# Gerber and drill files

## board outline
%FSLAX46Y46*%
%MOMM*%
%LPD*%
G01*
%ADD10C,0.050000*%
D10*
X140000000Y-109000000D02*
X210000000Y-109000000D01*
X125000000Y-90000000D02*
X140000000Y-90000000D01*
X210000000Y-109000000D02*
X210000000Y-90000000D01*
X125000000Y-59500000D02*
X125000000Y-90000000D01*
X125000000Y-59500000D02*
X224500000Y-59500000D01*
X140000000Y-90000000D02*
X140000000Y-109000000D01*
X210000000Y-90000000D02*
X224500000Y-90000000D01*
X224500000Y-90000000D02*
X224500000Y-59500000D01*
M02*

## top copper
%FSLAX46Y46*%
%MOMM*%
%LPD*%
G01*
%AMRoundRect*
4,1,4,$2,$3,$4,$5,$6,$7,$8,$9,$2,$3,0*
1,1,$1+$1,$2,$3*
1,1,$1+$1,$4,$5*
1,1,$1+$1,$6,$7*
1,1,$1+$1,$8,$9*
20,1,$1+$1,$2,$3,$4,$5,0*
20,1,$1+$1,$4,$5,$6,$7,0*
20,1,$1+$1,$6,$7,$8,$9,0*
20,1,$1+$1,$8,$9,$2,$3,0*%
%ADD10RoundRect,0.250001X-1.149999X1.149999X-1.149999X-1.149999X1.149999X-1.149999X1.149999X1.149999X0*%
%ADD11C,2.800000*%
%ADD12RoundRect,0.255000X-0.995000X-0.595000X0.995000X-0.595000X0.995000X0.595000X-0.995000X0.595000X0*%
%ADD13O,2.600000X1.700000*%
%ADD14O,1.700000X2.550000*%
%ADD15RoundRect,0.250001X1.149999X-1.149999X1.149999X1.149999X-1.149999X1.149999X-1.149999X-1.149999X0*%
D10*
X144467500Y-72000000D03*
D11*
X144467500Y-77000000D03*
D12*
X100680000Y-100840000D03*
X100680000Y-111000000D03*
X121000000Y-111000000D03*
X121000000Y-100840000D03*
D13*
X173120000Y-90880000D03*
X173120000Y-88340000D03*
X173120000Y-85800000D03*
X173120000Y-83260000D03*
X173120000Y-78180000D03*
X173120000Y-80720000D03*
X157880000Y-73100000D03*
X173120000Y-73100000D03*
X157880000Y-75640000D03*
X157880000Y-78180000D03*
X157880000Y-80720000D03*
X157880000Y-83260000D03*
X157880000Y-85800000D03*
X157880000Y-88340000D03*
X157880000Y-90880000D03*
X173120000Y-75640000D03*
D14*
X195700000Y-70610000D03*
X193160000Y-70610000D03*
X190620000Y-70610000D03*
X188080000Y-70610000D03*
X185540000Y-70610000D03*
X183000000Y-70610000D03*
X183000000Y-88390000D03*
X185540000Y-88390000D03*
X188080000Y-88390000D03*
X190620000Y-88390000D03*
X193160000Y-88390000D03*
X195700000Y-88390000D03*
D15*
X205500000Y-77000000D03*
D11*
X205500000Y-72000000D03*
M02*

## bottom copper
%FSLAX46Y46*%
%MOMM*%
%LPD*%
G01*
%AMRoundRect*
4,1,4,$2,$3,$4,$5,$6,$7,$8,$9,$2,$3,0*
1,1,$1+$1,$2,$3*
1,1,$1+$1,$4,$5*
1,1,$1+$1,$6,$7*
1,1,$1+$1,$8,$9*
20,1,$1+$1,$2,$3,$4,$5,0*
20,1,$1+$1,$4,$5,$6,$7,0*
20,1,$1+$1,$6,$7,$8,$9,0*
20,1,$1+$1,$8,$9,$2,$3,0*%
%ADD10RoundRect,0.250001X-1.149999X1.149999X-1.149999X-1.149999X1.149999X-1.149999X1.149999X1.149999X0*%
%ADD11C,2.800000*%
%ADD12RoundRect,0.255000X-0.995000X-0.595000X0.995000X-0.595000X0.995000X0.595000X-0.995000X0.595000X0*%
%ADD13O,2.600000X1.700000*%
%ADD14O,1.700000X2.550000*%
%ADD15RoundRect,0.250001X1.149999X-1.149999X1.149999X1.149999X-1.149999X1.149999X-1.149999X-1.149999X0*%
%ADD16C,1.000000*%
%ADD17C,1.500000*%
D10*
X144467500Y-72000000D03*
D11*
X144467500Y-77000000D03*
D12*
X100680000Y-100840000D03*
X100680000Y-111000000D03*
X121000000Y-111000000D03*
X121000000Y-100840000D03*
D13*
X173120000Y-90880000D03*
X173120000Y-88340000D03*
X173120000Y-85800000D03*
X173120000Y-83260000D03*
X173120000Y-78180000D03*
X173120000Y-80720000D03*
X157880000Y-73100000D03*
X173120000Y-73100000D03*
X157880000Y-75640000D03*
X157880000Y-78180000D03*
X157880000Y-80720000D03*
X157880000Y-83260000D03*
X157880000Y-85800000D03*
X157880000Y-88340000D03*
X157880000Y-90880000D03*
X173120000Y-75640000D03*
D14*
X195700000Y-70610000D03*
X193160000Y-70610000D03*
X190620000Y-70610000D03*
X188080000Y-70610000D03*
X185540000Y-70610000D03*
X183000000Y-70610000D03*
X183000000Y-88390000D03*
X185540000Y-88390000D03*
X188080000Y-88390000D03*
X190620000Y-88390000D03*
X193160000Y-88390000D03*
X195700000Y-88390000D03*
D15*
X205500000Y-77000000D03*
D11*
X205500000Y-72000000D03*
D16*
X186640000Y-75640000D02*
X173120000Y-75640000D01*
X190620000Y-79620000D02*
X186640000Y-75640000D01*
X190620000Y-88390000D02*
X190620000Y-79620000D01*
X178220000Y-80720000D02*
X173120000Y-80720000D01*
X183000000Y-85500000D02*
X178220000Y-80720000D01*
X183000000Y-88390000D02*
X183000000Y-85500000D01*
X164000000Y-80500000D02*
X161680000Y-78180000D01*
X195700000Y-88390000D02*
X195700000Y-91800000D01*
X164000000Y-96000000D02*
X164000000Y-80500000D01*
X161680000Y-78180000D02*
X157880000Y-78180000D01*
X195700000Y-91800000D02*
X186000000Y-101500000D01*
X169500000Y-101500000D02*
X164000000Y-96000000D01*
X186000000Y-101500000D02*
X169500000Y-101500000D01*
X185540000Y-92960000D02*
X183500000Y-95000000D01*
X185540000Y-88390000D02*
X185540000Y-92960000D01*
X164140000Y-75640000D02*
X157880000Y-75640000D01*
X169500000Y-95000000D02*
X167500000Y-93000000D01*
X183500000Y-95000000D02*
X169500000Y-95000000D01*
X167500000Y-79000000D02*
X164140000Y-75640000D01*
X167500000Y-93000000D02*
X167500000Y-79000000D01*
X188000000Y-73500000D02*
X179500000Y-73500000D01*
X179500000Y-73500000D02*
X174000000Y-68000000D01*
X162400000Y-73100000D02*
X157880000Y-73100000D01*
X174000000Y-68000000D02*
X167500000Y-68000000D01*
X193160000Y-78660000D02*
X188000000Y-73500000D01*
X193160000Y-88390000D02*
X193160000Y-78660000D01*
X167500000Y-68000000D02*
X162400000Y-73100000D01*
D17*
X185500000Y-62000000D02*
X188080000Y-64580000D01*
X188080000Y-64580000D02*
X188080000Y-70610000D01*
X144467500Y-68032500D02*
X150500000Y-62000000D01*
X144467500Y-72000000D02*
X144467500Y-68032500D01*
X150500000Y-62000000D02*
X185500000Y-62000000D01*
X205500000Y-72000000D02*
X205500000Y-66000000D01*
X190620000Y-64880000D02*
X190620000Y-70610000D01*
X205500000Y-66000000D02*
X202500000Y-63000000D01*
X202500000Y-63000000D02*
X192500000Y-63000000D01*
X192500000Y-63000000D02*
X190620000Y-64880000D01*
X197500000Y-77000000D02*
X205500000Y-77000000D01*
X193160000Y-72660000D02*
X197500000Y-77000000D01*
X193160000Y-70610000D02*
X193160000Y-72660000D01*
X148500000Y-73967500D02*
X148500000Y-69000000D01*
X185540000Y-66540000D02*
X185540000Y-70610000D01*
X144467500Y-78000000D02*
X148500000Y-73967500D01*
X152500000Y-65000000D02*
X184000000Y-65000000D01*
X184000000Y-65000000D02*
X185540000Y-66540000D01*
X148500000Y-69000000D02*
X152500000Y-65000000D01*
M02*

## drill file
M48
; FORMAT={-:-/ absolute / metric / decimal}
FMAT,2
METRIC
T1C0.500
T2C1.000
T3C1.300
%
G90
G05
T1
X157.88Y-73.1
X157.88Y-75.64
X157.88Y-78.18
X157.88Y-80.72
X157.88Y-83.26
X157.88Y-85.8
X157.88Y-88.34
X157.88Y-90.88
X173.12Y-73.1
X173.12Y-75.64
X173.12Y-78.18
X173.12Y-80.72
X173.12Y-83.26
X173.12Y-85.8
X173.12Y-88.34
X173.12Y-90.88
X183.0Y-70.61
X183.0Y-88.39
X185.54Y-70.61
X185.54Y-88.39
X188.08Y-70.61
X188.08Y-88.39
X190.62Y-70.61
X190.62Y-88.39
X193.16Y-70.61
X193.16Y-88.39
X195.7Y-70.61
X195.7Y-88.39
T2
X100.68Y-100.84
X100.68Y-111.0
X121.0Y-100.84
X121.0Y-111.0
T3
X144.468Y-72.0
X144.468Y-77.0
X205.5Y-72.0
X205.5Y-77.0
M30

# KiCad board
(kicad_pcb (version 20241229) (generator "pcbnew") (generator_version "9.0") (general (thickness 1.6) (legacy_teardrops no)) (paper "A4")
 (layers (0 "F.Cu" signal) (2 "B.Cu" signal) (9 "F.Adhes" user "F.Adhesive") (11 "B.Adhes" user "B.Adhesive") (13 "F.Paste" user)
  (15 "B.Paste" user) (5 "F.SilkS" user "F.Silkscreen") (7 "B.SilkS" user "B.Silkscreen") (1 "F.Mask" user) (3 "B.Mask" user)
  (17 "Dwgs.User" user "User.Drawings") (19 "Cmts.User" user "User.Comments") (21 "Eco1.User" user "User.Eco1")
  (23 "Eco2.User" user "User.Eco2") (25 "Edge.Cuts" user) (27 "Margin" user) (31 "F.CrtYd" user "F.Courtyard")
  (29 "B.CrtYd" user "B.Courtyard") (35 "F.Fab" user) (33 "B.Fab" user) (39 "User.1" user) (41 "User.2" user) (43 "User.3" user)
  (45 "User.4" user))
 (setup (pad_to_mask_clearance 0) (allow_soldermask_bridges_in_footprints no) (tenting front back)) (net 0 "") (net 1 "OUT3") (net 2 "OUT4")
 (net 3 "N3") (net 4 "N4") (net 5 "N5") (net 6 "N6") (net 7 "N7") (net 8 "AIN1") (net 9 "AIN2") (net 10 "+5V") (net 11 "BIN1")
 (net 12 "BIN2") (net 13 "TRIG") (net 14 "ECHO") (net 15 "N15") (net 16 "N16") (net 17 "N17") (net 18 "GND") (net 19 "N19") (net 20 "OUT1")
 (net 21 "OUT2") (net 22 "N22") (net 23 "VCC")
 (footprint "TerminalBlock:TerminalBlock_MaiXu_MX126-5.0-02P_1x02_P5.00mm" (layer "F.Cu") (at 144.4675 72 -90)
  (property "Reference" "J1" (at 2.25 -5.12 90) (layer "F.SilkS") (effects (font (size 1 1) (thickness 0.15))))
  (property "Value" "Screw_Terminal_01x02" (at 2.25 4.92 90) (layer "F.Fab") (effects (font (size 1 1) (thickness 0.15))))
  (pad "1" thru_hole roundrect (at 0 0 270) (size 2.8 2.8) (drill 1.3) (layers "*.Cu" "*.Mask") (remove_unused_layers no)
   (roundrect_rratio 0.089286) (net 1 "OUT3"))
  (pad "2" thru_hole circle (at 5 0 270) (size 2.8 2.8) (drill 1.3) (layers "*.Cu" "*.Mask") (remove_unused_layers no) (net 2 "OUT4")))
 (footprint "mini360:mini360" (layer "F.Cu") (at 110.84 103.38)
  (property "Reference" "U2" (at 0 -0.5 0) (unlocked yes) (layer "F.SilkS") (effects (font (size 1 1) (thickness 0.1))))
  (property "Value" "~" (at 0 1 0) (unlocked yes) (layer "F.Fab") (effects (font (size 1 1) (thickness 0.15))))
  (pad "1" thru_hole roundrect (at -10.16 -2.54) (size 2.5 1.7) (drill 1) (layers "*.Cu" "*.Mask") (remove_unused_layers no)
   (roundrect_rratio 0.15) (thermal_bridge_angle 45))
  (pad "2" thru_hole roundrect (at -10.16 7.62) (size 2.5 1.7) (drill 1) (layers "*.Cu" "*.Mask") (remove_unused_layers no)
   (roundrect_rratio 0.15) (thermal_bridge_angle 45))
  (pad "3" thru_hole roundrect (at 10.16 7.62) (size 2.5 1.7) (drill 1) (layers "*.Cu" "*.Mask") (remove_unused_layers no)
   (roundrect_rratio 0.15) (thermal_bridge_angle 45))
  (pad "4" thru_hole roundrect (at 10.16 -2.54) (size 2.5 1.7) (drill 1) (layers "*.Cu" "*.Mask") (remove_unused_layers no)
   (roundrect_rratio 0.15) (thermal_bridge_angle 45)))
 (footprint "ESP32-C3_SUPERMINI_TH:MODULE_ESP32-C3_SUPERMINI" (layer "F.Cu") (at 165.5 83)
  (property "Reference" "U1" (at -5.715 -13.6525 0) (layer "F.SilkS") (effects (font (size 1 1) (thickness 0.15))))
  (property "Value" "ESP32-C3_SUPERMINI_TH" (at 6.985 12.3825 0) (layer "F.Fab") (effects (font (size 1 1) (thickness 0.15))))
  (pad "0" thru_hole oval (at 7.62 7.88) (size 2.6 1.7) (drill 0.5) (layers "*.Cu" "*.Mask") (remove_unused_layers no) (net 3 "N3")
   (solder_mask_margin 0.102))
  (pad "1" thru_hole oval (at 7.62 5.34) (size 2.6 1.7) (drill 0.5) (layers "*.Cu" "*.Mask") (remove_unused_layers no) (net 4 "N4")
   (solder_mask_margin 0.102))
  (pad "2" thru_hole oval (at 7.62 2.8) (size 2.6 1.7) (drill 0.5) (layers "*.Cu" "*.Mask") (remove_unused_layers no) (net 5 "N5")
   (solder_mask_margin 0.102))
  (pad "3" thru_hole oval (at 7.62 0.26) (size 2.6 1.7) (drill 0.5) (layers "*.Cu" "*.Mask") (remove_unused_layers no) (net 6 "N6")
   (solder_mask_margin 0.102))
  (pad "3.3" thru_hole oval (at 7.62 -4.82) (size 2.6 1.7) (drill 0.5) (layers "*.Cu" "*.Mask") (remove_unused_layers no) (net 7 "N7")
   (solder_mask_margin 0.102))
  (pad "4" thru_hole oval (at 7.62 -2.28) (size 2.6 1.7) (drill 0.5) (layers "*.Cu" "*.Mask") (remove_unused_layers no) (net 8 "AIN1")
   (solder_mask_margin 0.102))
  (pad "5" thru_hole oval (at -7.62 -9.9) (size 2.6 1.7) (drill 0.5) (layers "*.Cu" "*.Mask") (remove_unused_layers no) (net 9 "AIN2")
   (solder_mask_margin 0.102))
  (pad "5V" thru_hole oval (at 7.62 -9.9) (size 2.6 1.7) (drill 0.5) (layers "*.Cu" "*.Mask") (remove_unused_layers no) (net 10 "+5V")
   (solder_mask_margin 0.102))
  (pad "6" thru_hole oval (at -7.62 -7.36) (size 2.6 1.7) (drill 0.5) (layers "*.Cu" "*.Mask") (remove_unused_layers no) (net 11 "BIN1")
   (solder_mask_margin 0.102))
  (pad "7" thru_hole oval (at -7.62 -4.82) (size 2.6 1.7) (drill 0.5) (layers "*.Cu" "*.Mask") (remove_unused_layers no) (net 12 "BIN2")
   (solder_mask_margin 0.102))
  (pad "8" thru_hole oval (at -7.62 -2.28) (size 2.6 1.7) (drill 0.5) (layers "*.Cu" "*.Mask") (remove_unused_layers no) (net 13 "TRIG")
   (solder_mask_margin 0.102))
  (pad "9" thru_hole oval (at -7.62 0.26) (size 2.6 1.7) (drill 0.5) (layers "*.Cu" "*.Mask") (remove_unused_layers no) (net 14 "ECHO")
   (solder_mask_margin 0.102))
  (pad "10" thru_hole oval (at -7.62 2.8) (size 2.6 1.7) (drill 0.5) (layers "*.Cu" "*.Mask") (remove_unused_layers no) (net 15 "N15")
   (solder_mask_margin 0.102))
  (pad "20" thru_hole oval (at -7.62 5.34) (size 2.6 1.7) (drill 0.5) (layers "*.Cu" "*.Mask") (remove_unused_layers no) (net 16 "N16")
   (solder_mask_margin 0.102))
  (pad "21" thru_hole oval (at -7.62 7.88) (size 2.6 1.7) (drill 0.5) (layers "*.Cu" "*.Mask") (remove_unused_layers no) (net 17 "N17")
   (solder_mask_margin 0.102))
  (pad "G" thru_hole oval (at 7.62 -7.36) (size 2.6 1.7) (drill 0.5) (layers "*.Cu" "*.Mask") (remove_unused_layers no) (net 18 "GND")
   (solder_mask_margin 0.102)))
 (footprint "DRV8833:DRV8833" (layer "F.Cu") (at 188.08 80.77 -90)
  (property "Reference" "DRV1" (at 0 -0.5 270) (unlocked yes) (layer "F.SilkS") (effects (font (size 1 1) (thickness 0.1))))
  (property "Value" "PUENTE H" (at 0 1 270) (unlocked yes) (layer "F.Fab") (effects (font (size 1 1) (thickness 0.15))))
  (pad "1" thru_hole oval (at -10.16 -7.62 270) (size 2.55 1.7) (drill 0.5) (layers "*.Cu" "*.Mask") (remove_unused_layers no)
   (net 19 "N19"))
  (pad "2" thru_hole oval (at -10.16 -5.08 270) (size 2.55 1.7) (drill 0.5) (layers "*.Cu" "*.Mask") (remove_unused_layers no)
   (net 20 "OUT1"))
  (pad "3" thru_hole oval (at -10.16 -2.54 270) (size 2.55 1.7) (drill 0.5) (layers "*.Cu" "*.Mask") (remove_unused_layers no)
   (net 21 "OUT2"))
  (pad "4" thru_hole oval (at -10.16 0 270) (size 2.55 1.7) (drill 0.5) (layers "*.Cu" "*.Mask") (remove_unused_layers no) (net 1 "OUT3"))
  (pad "5" thru_hole oval (at -10.16 2.54 270) (size 2.55 1.7) (drill 0.5) (layers "*.Cu" "*.Mask") (remove_unused_layers no) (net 2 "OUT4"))
  (pad "6" thru_hole oval (at -10.16 5.08 270) (size 2.55 1.7) (drill 0.5) (layers "*.Cu" "*.Mask") (remove_unused_layers no) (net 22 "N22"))
  (pad "7" thru_hole oval (at 7.62 5.08 270) (size 2.55 1.7) (drill 0.5) (layers "*.Cu" "*.Mask") (remove_unused_layers no) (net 8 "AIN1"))
  (pad "8" thru_hole oval (at 7.62 2.54 270) (size 2.55 1.7) (drill 0.5) (layers "*.Cu" "*.Mask") (remove_unused_layers no) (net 11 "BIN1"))
  (pad "9" thru_hole oval (at 7.62 0 270) (size 2.55 1.7) (drill 0.5) (layers "*.Cu" "*.Mask") (remove_unused_layers no) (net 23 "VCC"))
  (pad "10" thru_hole oval (at 7.62 -2.54 270) (size 2.55 1.7) (drill 0.5) (layers "*.Cu" "*.Mask") (remove_unused_layers no) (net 18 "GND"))
  (pad "11" thru_hole oval (at 7.62 -5.08 270) (size 2.55 1.7) (drill 0.5) (layers "*.Cu" "*.Mask") (remove_unused_layers no) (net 9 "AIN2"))
  (pad "12" thru_hole oval (at 7.62 -7.62 270) (size 2.55 1.7) (drill 0.5) (layers "*.Cu" "*.Mask") (remove_unused_layers no)
   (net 12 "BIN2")))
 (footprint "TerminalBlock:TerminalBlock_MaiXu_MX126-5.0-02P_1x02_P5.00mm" (layer "F.Cu") (at 205.5 77 90)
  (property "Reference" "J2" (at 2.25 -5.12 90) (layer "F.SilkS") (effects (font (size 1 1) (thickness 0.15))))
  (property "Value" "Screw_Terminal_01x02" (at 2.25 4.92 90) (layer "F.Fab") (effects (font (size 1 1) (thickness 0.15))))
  (pad "1" thru_hole roundrect (at 0 0 90) (size 2.8 2.8) (drill 1.3) (layers "*.Cu" "*.Mask") (remove_unused_layers no)
   (roundrect_rratio 0.089286) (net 20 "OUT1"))
  (pad "2" thru_hole circle (at 5 0 90) (size 2.8 2.8) (drill 1.3) (layers "*.Cu" "*.Mask") (remove_unused_layers no) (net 21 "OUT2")))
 (gr_line (start 140 109) (end 210 109) (stroke (width 0.05) (type default)) (layer "Edge.Cuts"))
 (gr_line (start 125 90) (end 140 90) (stroke (width 0.05) (type default)) (layer "Edge.Cuts"))
 (gr_line (start 210 109) (end 210 90) (stroke (width 0.05) (type default)) (layer "Edge.Cuts"))
 (gr_line (start 125 59.5) (end 125 90) (stroke (width 0.05) (type default)) (layer "Edge.Cuts"))
 (gr_line (start 125 59.5) (end 224.5 59.5) (stroke (width 0.05) (type default)) (layer "Edge.Cuts"))
 (gr_line (start 140 90) (end 140 109) (stroke (width 0.05) (type default)) (layer "Edge.Cuts"))
 (gr_line (start 210 90) (end 224.5 90) (stroke (width 0.05) (type default)) (layer "Edge.Cuts"))
 (gr_line (start 224.5 90) (end 224.5 59.5) (stroke (width 0.05) (type default)) (layer "Edge.Cuts"))
 (segment (start 186.64 75.64) (end 173.12 75.64) (width 1) (layer "B.Cu") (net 18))
 (segment (start 190.62 79.62) (end 186.64 75.64) (width 1) (layer "B.Cu") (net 18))
 (segment (start 190.62 88.39) (end 190.62 79.62) (width 1) (layer "B.Cu") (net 18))
 (segment (start 178.22 80.72) (end 173.12 80.72) (width 1) (layer "B.Cu") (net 8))
 (segment (start 183 85.5) (end 178.22 80.72) (width 1) (layer "B.Cu") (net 8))
 (segment (start 183 88.39) (end 183 85.5) (width 1) (layer "B.Cu") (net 8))
 (segment (start 164 80.5) (end 161.68 78.18) (width 1) (layer "B.Cu") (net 12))
 (segment (start 195.7 88.39) (end 195.7 91.8) (width 1) (layer "B.Cu") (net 12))
 (segment (start 164 96) (end 164 80.5) (width 1) (layer "B.Cu") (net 12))
 (segment (start 161.68 78.18) (end 157.88 78.18) (width 1) (layer "B.Cu") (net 12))
 (segment (start 195.7 91.8) (end 186 101.5) (width 1) (layer "B.Cu") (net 12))
 (segment (start 169.5 101.5) (end 164 96) (width 1) (layer "B.Cu") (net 12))
 (segment (start 186 101.5) (end 169.5 101.5) (width 1) (layer "B.Cu") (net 12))
 (segment (start 185.54 92.96) (end 183.5 95) (width 1) (layer "B.Cu") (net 11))
 (segment (start 185.54 88.39) (end 185.54 92.96) (width 1) (layer "B.Cu") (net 11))
 (segment (start 164.14 75.64) (end 157.88 75.64) (width 1) (layer "B.Cu") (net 11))
 (segment (start 169.5 95) (end 167.5 93) (width 1) (layer "B.Cu") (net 11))
 (segment (start 183.5 95) (end 169.5 95) (width 1) (layer "B.Cu") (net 11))
 (segment (start 167.5 79) (end 164.14 75.64) (width 1) (layer "B.Cu") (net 11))
 (segment (start 167.5 93) (end 167.5 79) (width 1) (layer "B.Cu") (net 11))
 (segment (start 188 73.5) (end 179.5 73.5) (width 1) (layer "B.Cu") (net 9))
 (segment (start 179.5 73.5) (end 174 68) (width 1) (layer "B.Cu") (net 9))
 (segment (start 162.4 73.1) (end 157.88 73.1) (width 1) (layer "B.Cu") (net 9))
 (segment (start 174 68) (end 167.5 68) (width 1) (layer "B.Cu") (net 9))
 (segment (start 193.16 78.66) (end 188 73.5) (width 1) (layer "B.Cu") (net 9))
 (segment (start 193.16 88.39) (end 193.16 78.66) (width 1) (layer "B.Cu") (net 9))
 (segment (start 167.5 68) (end 162.4 73.1) (width 1) (layer "B.Cu") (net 9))
 (segment (start 185.5 62) (end 188.08 64.58) (width 1.5) (layer "B.Cu") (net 1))
 (segment (start 188.08 64.58) (end 188.08 70.61) (width 1.5) (layer "B.Cu") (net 1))
 (segment (start 144.4675 68.0325) (end 150.5 62) (width 1.5) (layer "B.Cu") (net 1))
 (segment (start 144.4675 72) (end 144.4675 68.0325) (width 1.5) (layer "B.Cu") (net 1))
 (segment (start 150.5 62) (end 185.5 62) (width 1.5) (layer "B.Cu") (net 1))
 (segment (start 205.5 72) (end 205.5 66) (width 1.5) (layer "B.Cu") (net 21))
 (segment (start 190.62 64.88) (end 190.62 70.61) (width 1.5) (layer "B.Cu") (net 21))
 (segment (start 205.5 66) (end 202.5 63) (width 1.5) (layer "B.Cu") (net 21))
 (segment (start 202.5 63) (end 192.5 63) (width 1.5) (layer "B.Cu") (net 21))
 (segment (start 192.5 63) (end 190.62 64.88) (width 1.5) (layer "B.Cu") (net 21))
 (segment (start 197.5 77) (end 205.5 77) (width 1.5) (layer "B.Cu") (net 20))
 (segment (start 193.16 72.66) (end 197.5 77) (width 1.5) (layer "B.Cu") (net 20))
 (segment (start 193.16 70.61) (end 193.16 72.66) (width 1.5) (layer "B.Cu") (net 20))
 (segment (start 148.5 73.9675) (end 148.5 69) (width 1.5) (layer "B.Cu") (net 2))
 (segment (start 185.54 66.54) (end 185.54 70.61) (width 1.5) (layer "B.Cu") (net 2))
 (segment (start 144.4675 78) (end 148.5 73.9675) (width 1.5) (layer "B.Cu") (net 2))
 (segment (start 152.5 65) (end 184 65) (width 1.5) (layer "B.Cu") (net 2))
 (segment (start 184 65) (end 185.54 66.54) (width 1.5) (layer "B.Cu") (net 2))
 (segment (start 148.5 69) (end 152.5 65) (width 1.5) (layer "B.Cu") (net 2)))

